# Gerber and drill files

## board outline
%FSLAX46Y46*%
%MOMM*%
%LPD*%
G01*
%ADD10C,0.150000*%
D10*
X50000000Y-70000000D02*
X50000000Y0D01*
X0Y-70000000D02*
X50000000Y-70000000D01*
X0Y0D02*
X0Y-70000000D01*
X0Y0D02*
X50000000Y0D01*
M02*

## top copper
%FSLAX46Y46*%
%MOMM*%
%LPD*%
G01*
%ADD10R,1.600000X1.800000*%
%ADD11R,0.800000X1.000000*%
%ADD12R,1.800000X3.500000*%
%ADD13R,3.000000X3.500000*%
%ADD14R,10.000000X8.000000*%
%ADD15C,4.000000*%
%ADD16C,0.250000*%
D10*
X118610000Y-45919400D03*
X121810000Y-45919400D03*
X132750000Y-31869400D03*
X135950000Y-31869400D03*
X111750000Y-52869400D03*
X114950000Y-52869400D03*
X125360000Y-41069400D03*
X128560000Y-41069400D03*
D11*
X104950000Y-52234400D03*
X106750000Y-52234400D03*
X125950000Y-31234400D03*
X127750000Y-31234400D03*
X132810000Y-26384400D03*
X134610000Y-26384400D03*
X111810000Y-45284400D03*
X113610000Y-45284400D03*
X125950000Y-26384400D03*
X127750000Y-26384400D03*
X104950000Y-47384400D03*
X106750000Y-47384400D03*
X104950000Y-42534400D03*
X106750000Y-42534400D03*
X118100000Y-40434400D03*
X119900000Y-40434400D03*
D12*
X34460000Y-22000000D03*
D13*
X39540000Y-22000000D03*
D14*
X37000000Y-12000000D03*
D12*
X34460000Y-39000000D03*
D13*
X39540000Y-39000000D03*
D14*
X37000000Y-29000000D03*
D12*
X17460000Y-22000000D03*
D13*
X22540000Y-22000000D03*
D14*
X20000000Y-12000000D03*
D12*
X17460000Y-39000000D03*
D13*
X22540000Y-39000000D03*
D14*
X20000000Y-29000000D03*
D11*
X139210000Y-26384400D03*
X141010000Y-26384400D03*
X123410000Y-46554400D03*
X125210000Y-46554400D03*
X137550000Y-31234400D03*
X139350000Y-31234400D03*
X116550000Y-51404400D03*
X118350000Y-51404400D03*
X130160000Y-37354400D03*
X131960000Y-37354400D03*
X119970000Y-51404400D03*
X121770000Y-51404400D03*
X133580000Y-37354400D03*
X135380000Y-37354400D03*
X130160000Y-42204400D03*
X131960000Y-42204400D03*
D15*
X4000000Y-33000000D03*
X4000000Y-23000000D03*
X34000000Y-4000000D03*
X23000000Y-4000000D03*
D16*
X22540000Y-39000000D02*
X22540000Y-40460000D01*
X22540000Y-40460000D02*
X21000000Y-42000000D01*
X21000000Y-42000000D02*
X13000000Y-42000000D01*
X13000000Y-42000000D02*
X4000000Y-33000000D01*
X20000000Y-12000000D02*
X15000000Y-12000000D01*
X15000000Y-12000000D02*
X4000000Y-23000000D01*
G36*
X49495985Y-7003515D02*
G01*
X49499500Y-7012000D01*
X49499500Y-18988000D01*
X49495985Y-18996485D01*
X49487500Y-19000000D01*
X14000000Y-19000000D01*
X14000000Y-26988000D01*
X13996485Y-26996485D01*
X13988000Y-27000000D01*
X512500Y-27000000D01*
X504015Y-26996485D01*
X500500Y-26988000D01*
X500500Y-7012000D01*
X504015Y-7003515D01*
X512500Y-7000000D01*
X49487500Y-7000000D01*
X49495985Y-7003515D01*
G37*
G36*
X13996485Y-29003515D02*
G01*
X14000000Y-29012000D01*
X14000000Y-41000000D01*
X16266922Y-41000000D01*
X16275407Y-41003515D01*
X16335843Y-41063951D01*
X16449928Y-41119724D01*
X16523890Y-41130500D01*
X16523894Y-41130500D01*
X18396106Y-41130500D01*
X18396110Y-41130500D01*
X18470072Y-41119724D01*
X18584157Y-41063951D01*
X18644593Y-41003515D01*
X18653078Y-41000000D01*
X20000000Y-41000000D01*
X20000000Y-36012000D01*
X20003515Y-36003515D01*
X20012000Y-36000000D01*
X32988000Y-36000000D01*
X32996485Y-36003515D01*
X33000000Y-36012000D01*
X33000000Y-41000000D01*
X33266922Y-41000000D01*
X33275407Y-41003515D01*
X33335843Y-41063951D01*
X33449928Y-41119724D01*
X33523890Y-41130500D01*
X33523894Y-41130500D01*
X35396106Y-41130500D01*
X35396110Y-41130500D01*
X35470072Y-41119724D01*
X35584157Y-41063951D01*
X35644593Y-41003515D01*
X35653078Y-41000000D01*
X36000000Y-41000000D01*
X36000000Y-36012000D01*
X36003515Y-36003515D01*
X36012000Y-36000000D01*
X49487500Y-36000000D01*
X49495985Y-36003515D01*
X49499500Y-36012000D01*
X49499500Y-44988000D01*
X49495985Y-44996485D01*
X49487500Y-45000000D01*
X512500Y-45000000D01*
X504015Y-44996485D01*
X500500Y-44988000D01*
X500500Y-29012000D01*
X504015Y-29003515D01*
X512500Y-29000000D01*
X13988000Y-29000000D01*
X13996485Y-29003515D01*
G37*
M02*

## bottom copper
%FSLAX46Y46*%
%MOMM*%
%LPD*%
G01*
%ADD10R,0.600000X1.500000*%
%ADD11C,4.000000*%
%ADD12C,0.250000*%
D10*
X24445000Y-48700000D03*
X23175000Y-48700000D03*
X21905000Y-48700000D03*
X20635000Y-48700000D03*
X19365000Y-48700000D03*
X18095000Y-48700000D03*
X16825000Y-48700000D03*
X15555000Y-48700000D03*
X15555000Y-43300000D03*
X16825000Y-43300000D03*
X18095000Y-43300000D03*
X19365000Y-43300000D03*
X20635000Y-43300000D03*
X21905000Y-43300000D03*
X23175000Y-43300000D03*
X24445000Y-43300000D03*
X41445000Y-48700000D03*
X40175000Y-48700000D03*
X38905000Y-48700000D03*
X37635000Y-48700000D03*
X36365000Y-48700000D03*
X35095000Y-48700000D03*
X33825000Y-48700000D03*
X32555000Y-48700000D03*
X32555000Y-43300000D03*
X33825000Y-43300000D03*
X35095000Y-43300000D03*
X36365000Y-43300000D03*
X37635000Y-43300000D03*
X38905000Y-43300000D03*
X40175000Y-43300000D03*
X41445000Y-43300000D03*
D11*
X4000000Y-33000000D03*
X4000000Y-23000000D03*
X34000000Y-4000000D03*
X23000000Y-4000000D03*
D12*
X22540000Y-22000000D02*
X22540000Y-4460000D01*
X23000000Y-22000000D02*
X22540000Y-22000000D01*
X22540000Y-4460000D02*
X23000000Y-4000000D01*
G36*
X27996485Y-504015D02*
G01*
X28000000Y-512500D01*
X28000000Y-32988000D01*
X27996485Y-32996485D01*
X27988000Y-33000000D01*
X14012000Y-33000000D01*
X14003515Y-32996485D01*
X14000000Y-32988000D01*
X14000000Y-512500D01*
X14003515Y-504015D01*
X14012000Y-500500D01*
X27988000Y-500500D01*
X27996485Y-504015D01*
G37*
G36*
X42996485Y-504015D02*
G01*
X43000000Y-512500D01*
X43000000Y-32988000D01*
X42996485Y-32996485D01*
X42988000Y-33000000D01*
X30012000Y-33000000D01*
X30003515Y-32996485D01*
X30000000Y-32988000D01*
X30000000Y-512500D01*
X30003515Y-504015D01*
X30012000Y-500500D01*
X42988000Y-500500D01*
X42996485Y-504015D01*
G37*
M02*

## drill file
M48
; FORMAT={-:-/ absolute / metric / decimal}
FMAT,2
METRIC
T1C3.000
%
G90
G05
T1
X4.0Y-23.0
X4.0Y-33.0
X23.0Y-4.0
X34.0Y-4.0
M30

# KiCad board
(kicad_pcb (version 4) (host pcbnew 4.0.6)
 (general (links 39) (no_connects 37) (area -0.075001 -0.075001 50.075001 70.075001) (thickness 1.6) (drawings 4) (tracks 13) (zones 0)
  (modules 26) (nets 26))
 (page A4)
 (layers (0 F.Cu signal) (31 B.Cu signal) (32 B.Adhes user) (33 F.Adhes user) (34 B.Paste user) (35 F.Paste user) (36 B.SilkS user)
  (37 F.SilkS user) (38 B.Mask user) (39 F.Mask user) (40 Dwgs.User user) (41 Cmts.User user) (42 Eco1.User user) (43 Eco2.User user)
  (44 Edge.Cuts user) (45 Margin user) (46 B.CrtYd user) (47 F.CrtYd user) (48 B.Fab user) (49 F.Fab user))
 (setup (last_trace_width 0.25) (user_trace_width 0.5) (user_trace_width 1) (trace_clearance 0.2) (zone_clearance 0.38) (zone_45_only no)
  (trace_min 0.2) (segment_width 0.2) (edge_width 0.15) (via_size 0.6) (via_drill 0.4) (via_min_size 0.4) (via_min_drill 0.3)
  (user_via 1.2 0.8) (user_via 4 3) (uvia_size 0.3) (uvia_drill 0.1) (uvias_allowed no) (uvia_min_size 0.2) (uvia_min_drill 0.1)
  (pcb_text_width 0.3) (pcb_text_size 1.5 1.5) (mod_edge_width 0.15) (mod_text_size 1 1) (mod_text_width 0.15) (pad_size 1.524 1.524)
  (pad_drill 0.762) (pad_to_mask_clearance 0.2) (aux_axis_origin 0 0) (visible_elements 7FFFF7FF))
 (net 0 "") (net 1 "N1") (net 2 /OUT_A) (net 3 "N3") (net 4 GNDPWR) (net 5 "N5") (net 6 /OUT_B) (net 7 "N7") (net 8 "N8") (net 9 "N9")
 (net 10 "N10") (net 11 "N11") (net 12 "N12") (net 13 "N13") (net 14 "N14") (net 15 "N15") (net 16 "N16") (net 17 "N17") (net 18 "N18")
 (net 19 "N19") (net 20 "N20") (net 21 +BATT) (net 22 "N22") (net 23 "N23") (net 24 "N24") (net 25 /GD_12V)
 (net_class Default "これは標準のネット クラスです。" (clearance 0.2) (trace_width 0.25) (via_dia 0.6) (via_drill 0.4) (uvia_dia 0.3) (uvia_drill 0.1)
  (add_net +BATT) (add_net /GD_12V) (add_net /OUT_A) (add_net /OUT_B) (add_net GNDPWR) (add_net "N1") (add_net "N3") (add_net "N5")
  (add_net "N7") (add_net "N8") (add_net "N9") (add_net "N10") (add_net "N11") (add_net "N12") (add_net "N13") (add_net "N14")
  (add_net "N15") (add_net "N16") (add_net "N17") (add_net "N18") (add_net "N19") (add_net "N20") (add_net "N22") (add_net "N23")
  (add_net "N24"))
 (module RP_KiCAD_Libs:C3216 (layer F.Cu) (at 120.21 45.9194)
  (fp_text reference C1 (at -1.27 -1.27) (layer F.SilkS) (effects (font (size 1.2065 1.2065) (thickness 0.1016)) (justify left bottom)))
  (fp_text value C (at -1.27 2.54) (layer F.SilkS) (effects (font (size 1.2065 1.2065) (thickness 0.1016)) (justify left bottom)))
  (pad 1 smd rect (at -1.6 0) (size 1.6 1.8) (layers F.Cu F.Paste F.Mask) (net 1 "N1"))
  (pad 2 smd rect (at 1.6 0) (size 1.6 1.8) (layers F.Cu F.Paste F.Mask) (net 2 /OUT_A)))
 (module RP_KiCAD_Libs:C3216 (layer F.Cu) (at 134.35 31.8694)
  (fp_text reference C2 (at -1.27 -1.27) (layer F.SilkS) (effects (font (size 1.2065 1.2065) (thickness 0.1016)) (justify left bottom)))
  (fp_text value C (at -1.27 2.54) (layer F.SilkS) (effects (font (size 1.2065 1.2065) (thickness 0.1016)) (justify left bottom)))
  (pad 1 smd rect (at -1.6 0) (size 1.6 1.8) (layers F.Cu F.Paste F.Mask) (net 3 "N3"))
  (pad 2 smd rect (at 1.6 0) (size 1.6 1.8) (layers F.Cu F.Paste F.Mask) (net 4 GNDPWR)))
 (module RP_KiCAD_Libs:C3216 (layer F.Cu) (at 113.35 52.8694)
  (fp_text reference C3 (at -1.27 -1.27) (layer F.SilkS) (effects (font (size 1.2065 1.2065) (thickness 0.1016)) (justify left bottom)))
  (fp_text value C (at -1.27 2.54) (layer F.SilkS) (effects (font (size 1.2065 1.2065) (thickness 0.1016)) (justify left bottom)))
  (pad 1 smd rect (at -1.6 0) (size 1.6 1.8) (layers F.Cu F.Paste F.Mask) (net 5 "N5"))
  (pad 2 smd rect (at 1.6 0) (size 1.6 1.8) (layers F.Cu F.Paste F.Mask) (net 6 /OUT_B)))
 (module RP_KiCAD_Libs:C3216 (layer F.Cu) (at 126.96 41.0694)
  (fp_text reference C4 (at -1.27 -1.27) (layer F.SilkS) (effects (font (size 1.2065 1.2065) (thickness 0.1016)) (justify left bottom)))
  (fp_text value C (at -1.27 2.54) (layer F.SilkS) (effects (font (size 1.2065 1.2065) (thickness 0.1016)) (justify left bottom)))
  (pad 1 smd rect (at -1.6 0) (size 1.6 1.8) (layers F.Cu F.Paste F.Mask) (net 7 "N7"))
  (pad 2 smd rect (at 1.6 0) (size 1.6 1.8) (layers F.Cu F.Paste F.Mask) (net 4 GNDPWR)))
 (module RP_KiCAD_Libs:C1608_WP (layer F.Cu) (at 105.85 52.2344)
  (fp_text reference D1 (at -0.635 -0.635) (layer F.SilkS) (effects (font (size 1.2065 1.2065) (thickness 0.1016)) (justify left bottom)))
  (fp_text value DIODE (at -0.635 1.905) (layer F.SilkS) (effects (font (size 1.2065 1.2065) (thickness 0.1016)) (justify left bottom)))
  (pad 1 smd rect (at -0.9 0) (size 0.8 1) (layers F.Cu F.Paste F.Mask) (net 1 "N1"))
  (pad 2 smd rect (at 0.9 0) (size 0.8 1) (layers F.Cu F.Paste F.Mask) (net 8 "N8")))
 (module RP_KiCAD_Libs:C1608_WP (layer F.Cu) (at 126.85 31.2344)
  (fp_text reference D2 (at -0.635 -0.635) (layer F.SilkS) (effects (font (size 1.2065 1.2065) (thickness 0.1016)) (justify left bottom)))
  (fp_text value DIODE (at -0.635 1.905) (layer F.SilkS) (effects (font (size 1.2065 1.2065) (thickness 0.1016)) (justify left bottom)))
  (pad 1 smd rect (at -0.9 0) (size 0.8 1) (layers F.Cu F.Paste F.Mask) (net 3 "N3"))
  (pad 2 smd rect (at 0.9 0) (size 0.8 1) (layers F.Cu F.Paste F.Mask) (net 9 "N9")))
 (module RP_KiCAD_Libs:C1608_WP (layer F.Cu) (at 133.71 26.3844)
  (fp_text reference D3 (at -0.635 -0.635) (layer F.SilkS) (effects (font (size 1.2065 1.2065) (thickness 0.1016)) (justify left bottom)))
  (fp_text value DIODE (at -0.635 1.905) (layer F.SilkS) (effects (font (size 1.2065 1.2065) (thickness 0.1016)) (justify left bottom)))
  (pad 1 smd rect (at -0.9 0) (size 0.8 1) (layers F.Cu F.Paste F.Mask) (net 5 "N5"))
  (pad 2 smd rect (at 0.9 0) (size 0.8 1) (layers F.Cu F.Paste F.Mask) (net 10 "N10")))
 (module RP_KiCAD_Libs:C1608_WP (layer F.Cu) (at 112.71 45.2844)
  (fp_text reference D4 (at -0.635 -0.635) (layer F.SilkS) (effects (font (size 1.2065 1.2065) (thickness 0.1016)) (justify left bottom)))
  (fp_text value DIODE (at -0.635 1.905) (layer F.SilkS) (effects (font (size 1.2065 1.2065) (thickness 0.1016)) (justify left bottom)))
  (pad 1 smd rect (at -0.9 0) (size 0.8 1) (layers F.Cu F.Paste F.Mask) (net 7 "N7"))
  (pad 2 smd rect (at 0.9 0) (size 0.8 1) (layers F.Cu F.Paste F.Mask) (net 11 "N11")))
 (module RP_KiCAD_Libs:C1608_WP (layer F.Cu) (at 126.85 26.3844)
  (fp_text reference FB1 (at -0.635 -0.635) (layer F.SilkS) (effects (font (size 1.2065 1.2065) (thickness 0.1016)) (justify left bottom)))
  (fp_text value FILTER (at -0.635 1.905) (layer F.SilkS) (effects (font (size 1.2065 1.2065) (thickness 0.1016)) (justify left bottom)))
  (pad 1 smd rect (at -0.9 0) (size 0.8 1) (layers F.Cu F.Paste F.Mask) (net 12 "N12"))
  (pad 2 smd rect (at 0.9 0) (size 0.8 1) (layers F.Cu F.Paste F.Mask) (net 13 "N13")))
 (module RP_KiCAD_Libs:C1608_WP (layer F.Cu) (at 105.85 47.3844)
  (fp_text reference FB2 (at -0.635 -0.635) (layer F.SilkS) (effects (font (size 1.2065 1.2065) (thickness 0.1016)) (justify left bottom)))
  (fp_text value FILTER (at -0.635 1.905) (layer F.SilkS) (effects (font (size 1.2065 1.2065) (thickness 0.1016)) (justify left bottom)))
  (pad 1 smd rect (at -0.9 0) (size 0.8 1) (layers F.Cu F.Paste F.Mask) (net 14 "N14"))
  (pad 2 smd rect (at 0.9 0) (size 0.8 1) (layers F.Cu F.Paste F.Mask) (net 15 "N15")))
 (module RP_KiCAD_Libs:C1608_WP (layer F.Cu) (at 105.85 42.5344)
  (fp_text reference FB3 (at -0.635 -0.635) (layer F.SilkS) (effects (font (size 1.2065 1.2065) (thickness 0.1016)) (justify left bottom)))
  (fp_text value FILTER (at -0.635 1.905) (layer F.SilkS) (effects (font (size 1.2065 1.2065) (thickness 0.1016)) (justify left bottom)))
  (pad 1 smd rect (at -0.9 0) (size 0.8 1) (layers F.Cu F.Paste F.Mask) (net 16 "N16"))
  (pad 2 smd rect (at 0.9 0) (size 0.8 1) (layers F.Cu F.Paste F.Mask) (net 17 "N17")))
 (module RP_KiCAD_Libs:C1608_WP (layer F.Cu) (at 119 40.4344)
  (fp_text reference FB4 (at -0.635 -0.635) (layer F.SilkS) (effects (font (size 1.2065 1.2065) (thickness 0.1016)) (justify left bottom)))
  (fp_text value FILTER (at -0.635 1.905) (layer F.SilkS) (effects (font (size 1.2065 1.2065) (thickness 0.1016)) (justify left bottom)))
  (pad 1 smd rect (at -0.9 0) (size 0.8 1) (layers F.Cu F.Paste F.Mask) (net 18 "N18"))
  (pad 2 smd rect (at 0.9 0) (size 0.8 1) (layers F.Cu F.Paste F.Mask) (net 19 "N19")))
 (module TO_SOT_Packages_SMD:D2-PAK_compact (layer F.Cu) (at 37 19)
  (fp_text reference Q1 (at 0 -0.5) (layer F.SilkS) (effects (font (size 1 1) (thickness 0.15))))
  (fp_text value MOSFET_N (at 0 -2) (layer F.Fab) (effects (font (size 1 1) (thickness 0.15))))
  (pad G smd rect (at -2.54 3) (size 1.8 3.5) (layers F.Cu F.Paste F.Mask) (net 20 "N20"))
  (pad S smd rect (at 2.54 3) (size 3 3.5) (layers F.Cu F.Paste F.Mask) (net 2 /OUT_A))
  (pad D smd rect (at 0 -7) (size 10 8) (layers F.Cu F.Paste F.Mask) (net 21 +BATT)))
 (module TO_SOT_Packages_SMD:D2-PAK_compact (layer F.Cu) (at 37 36)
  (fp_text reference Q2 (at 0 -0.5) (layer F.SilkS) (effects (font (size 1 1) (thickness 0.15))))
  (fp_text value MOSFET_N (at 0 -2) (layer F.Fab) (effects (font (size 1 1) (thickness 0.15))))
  (pad G smd rect (at -2.54 3) (size 1.8 3.5) (layers F.Cu F.Paste F.Mask) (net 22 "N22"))
  (pad S smd rect (at 2.54 3) (size 3 3.5) (layers F.Cu F.Paste F.Mask) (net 4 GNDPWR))
  (pad D smd rect (at 0 -7) (size 10 8) (layers F.Cu F.Paste F.Mask) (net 2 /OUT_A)))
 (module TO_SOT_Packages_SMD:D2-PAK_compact (layer F.Cu) (at 20 19)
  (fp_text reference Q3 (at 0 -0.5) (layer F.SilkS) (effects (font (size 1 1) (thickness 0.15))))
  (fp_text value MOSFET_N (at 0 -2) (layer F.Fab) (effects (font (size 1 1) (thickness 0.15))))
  (pad G smd rect (at -2.54 3) (size 1.8 3.5) (layers F.Cu F.Paste F.Mask) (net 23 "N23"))
  (pad S smd rect (at 2.54 3) (size 3 3.5) (layers F.Cu F.Paste F.Mask) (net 6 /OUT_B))
  (pad D smd rect (at 0 -7) (size 10 8) (layers F.Cu F.Paste F.Mask) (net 21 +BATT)))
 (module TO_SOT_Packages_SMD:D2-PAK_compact (layer F.Cu) (at 20 36)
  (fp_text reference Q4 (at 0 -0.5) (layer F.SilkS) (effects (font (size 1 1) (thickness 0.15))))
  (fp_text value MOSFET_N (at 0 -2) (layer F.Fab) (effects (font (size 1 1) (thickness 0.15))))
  (pad G smd rect (at -2.54 3) (size 1.8 3.5) (layers F.Cu F.Paste F.Mask) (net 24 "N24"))
  (pad S smd rect (at 2.54 3) (size 3 3.5) (layers F.Cu F.Paste F.Mask) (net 4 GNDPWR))
  (pad D smd rect (at 0 -7) (size 10 8) (layers F.Cu F.Paste F.Mask) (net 6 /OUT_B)))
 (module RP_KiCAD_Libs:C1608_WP (layer F.Cu) (at 140.11 26.3844)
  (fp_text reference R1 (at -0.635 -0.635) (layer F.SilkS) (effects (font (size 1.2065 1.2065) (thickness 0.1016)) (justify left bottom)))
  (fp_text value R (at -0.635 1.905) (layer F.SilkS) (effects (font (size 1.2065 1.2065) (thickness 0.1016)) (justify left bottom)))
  (pad 1 smd rect (at -0.9 0) (size 0.8 1) (layers F.Cu F.Paste F.Mask) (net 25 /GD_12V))
  (pad 2 smd rect (at 0.9 0) (size 0.8 1) (layers F.Cu F.Paste F.Mask) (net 8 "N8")))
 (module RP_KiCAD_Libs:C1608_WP (layer F.Cu) (at 124.31 46.5544)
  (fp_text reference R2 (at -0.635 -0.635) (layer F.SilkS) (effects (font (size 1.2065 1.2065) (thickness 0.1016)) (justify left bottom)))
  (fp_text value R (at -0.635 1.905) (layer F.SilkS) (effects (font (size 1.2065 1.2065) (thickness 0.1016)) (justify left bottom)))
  (pad 1 smd rect (at -0.9 0) (size 0.8 1) (layers F.Cu F.Paste F.Mask) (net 25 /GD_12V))
  (pad 2 smd rect (at 0.9 0) (size 0.8 1) (layers F.Cu F.Paste F.Mask) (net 9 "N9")))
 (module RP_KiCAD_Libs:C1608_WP (layer F.Cu) (at 138.45 31.2344)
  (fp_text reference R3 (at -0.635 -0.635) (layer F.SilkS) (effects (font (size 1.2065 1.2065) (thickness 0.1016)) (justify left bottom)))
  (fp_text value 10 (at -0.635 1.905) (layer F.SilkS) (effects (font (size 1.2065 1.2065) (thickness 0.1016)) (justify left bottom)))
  (pad 1 smd rect (at -0.9 0) (size 0.8 1) (layers F.Cu F.Paste F.Mask) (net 20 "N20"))
  (pad 2 smd rect (at 0.9 0) (size 0.8 1) (layers F.Cu F.Paste F.Mask) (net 13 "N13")))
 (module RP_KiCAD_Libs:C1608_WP (layer F.Cu) (at 117.45 51.4044)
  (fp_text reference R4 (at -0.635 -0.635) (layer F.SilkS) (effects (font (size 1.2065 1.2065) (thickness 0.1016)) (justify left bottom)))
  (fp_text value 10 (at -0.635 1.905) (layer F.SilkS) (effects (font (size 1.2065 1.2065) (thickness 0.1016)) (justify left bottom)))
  (pad 1 smd rect (at -0.9 0) (size 0.8 1) (layers F.Cu F.Paste F.Mask) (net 22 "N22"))
  (pad 2 smd rect (at 0.9 0) (size 0.8 1) (layers F.Cu F.Paste F.Mask) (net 15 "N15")))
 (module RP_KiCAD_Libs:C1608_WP (layer F.Cu) (at 131.06 37.3544)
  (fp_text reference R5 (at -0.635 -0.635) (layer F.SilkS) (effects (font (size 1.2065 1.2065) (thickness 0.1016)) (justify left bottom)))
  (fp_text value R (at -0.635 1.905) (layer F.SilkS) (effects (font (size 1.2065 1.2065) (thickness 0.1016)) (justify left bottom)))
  (pad 1 smd rect (at -0.9 0) (size 0.8 1) (layers F.Cu F.Paste F.Mask) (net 25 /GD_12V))
  (pad 2 smd rect (at 0.9 0) (size 0.8 1) (layers F.Cu F.Paste F.Mask) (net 10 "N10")))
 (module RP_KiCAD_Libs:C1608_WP (layer F.Cu) (at 120.87 51.4044)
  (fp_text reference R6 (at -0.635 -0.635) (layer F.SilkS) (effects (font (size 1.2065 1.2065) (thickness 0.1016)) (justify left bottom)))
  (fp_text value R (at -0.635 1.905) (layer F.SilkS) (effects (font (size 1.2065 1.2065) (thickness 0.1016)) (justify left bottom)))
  (pad 1 smd rect (at -0.9 0) (size 0.8 1) (layers F.Cu F.Paste F.Mask) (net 25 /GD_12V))
  (pad 2 smd rect (at 0.9 0) (size 0.8 1) (layers F.Cu F.Paste F.Mask) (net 11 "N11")))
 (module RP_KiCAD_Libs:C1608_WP (layer F.Cu) (at 134.48 37.3544)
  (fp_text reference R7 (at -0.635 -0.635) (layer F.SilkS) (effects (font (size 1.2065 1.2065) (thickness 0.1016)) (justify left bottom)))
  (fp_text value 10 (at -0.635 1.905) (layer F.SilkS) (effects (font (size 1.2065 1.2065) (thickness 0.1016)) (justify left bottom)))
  (pad 1 smd rect (at -0.9 0) (size 0.8 1) (layers F.Cu F.Paste F.Mask) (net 23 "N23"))
  (pad 2 smd rect (at 0.9 0) (size 0.8 1) (layers F.Cu F.Paste F.Mask) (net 17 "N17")))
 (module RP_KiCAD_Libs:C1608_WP (layer F.Cu) (at 131.06 42.2044)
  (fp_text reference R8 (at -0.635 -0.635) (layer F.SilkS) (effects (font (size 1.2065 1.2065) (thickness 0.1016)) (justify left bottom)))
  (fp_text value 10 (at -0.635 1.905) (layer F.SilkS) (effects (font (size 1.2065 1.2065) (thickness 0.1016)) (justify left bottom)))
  (pad 1 smd rect (at -0.9 0) (size 0.8 1) (layers F.Cu F.Paste F.Mask) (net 24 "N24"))
  (pad 2 smd rect (at 0.9 0) (size 0.8 1) (layers F.Cu F.Paste F.Mask) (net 19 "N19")))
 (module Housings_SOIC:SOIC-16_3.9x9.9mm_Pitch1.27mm (layer B.Cu) (at 20 46 90)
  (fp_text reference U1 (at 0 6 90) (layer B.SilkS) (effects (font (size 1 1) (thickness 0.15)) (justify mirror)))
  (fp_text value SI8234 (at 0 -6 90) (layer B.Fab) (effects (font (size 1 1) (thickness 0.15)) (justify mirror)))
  (pad 1 smd rect (at -2.7 4.445 90) (size 1.5 0.6) (layers B.Cu B.Paste B.Mask))
  (pad 2 smd rect (at -2.7 3.175 90) (size 1.5 0.6) (layers B.Cu B.Paste B.Mask))
  (pad 3 smd rect (at -2.7 1.905 90) (size 1.5 0.6) (layers B.Cu B.Paste B.Mask))
  (pad 4 smd rect (at -2.7 0.635 90) (size 1.5 0.6) (layers B.Cu B.Paste B.Mask))
  (pad 5 smd rect (at -2.7 -0.635 90) (size 1.5 0.6) (layers B.Cu B.Paste B.Mask))
  (pad 6 smd rect (at -2.7 -1.905 90) (size 1.5 0.6) (layers B.Cu B.Paste B.Mask))
  (pad 7 smd rect (at -2.7 -3.175 90) (size 1.5 0.6) (layers B.Cu B.Paste B.Mask))
  (pad 8 smd rect (at -2.7 -4.445 90) (size 1.5 0.6) (layers B.Cu B.Paste B.Mask))
  (pad 9 smd rect (at 2.7 -4.445 90) (size 1.5 0.6) (layers B.Cu B.Paste B.Mask) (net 4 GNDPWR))
  (pad 10 smd rect (at 2.7 -3.175 90) (size 1.5 0.6) (layers B.Cu B.Paste B.Mask) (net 14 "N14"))
  (pad 11 smd rect (at 2.7 -1.905 90) (size 1.5 0.6) (layers B.Cu B.Paste B.Mask) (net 3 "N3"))
  (pad 12 smd rect (at 2.7 -0.635 90) (size 1.5 0.6) (layers B.Cu B.Paste B.Mask))
  (pad 13 smd rect (at 2.7 0.635 90) (size 1.5 0.6) (layers B.Cu B.Paste B.Mask))
  (pad 14 smd rect (at 2.7 1.905 90) (size 1.5 0.6) (layers B.Cu B.Paste B.Mask) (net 2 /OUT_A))
  (pad 15 smd rect (at 2.7 3.175 90) (size 1.5 0.6) (layers B.Cu B.Paste B.Mask) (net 12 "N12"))
  (pad 16 smd rect (at 2.7 4.445 90) (size 1.5 0.6) (layers B.Cu B.Paste B.Mask) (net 1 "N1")))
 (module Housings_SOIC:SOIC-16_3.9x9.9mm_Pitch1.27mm (layer B.Cu) (at 37 46 90)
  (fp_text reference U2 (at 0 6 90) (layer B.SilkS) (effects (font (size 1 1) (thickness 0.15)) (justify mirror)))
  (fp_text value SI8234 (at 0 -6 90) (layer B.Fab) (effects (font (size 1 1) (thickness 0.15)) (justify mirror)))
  (pad 1 smd rect (at -2.7 4.445 90) (size 1.5 0.6) (layers B.Cu B.Paste B.Mask))
  (pad 2 smd rect (at -2.7 3.175 90) (size 1.5 0.6) (layers B.Cu B.Paste B.Mask))
  (pad 3 smd rect (at -2.7 1.905 90) (size 1.5 0.6) (layers B.Cu B.Paste B.Mask))
  (pad 4 smd rect (at -2.7 0.635 90) (size 1.5 0.6) (layers B.Cu B.Paste B.Mask))
  (pad 5 smd rect (at -2.7 -0.635 90) (size 1.5 0.6) (layers B.Cu B.Paste B.Mask))
  (pad 6 smd rect (at -2.7 -1.905 90) (size 1.5 0.6) (layers B.Cu B.Paste B.Mask))
  (pad 7 smd rect (at -2.7 -3.175 90) (size 1.5 0.6) (layers B.Cu B.Paste B.Mask))
  (pad 8 smd rect (at -2.7 -4.445 90) (size 1.5 0.6) (layers B.Cu B.Paste B.Mask))
  (pad 9 smd rect (at 2.7 -4.445 90) (size 1.5 0.6) (layers B.Cu B.Paste B.Mask) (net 4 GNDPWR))
  (pad 10 smd rect (at 2.7 -3.175 90) (size 1.5 0.6) (layers B.Cu B.Paste B.Mask) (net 18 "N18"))
  (pad 11 smd rect (at 2.7 -1.905 90) (size 1.5 0.6) (layers B.Cu B.Paste B.Mask) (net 7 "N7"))
  (pad 12 smd rect (at 2.7 -0.635 90) (size 1.5 0.6) (layers B.Cu B.Paste B.Mask))
  (pad 13 smd rect (at 2.7 0.635 90) (size 1.5 0.6) (layers B.Cu B.Paste B.Mask))
  (pad 14 smd rect (at 2.7 1.905 90) (size 1.5 0.6) (layers B.Cu B.Paste B.Mask) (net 6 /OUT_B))
  (pad 15 smd rect (at 2.7 3.175 90) (size 1.5 0.6) (layers B.Cu B.Paste B.Mask) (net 16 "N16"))
  (pad 16 smd rect (at 2.7 4.445 90) (size 1.5 0.6) (layers B.Cu B.Paste B.Mask) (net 5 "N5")))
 (gr_line (start 50 70) (end 50 0) (angle 90) (layer Edge.Cuts) (width 0.15))
 (gr_line (start 0 70) (end 50 70) (angle 90) (layer Edge.Cuts) (width 0.15))
 (gr_line (start 0 0) (end 0 70) (angle 90) (layer Edge.Cuts) (width 0.15))
 (gr_line (start 0 0) (end 50 0) (angle 90) (layer Edge.Cuts) (width 0.15))
 (segment (start 22.54 39) (end 22.54 40.46) (width 0.25) (layer F.Cu) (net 4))
 (segment (start 22.54 40.46) (end 21 42) (width 0.25) (layer F.Cu) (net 4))
 (segment (start 21 42) (end 13 42) (width 0.25) (layer F.Cu) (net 4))
 (segment (start 13 42) (end 4 33) (width 0.25) (layer F.Cu) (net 4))
 (via (at 4 33) (size 4) (drill 3) (layers F.Cu B.Cu) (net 4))
 (segment (start 20 12) (end 15 12) (width 0.25) (layer F.Cu) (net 21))
 (segment (start 15 12) (end 4 23) (width 0.25) (layer F.Cu) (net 21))
 (via (at 4 23) (size 4) (drill 3) (layers F.Cu B.Cu) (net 21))
 (via (at 34 4) (size 4) (drill 3) (layers F.Cu B.Cu) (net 2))
 (segment (start 22.54 22) (end 22.54 4.46) (width 0.25) (layer B.Cu) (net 6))
 (segment (start 23 22) (end 22.54 22) (width 0.25) (layer B.Cu) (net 6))
 (via (at 23 4) (size 4) (drill 3) (layers F.Cu B.Cu) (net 6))
 (segment (start 22.54 4.46) (end 23 4) (width 0.25) (layer B.Cu) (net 6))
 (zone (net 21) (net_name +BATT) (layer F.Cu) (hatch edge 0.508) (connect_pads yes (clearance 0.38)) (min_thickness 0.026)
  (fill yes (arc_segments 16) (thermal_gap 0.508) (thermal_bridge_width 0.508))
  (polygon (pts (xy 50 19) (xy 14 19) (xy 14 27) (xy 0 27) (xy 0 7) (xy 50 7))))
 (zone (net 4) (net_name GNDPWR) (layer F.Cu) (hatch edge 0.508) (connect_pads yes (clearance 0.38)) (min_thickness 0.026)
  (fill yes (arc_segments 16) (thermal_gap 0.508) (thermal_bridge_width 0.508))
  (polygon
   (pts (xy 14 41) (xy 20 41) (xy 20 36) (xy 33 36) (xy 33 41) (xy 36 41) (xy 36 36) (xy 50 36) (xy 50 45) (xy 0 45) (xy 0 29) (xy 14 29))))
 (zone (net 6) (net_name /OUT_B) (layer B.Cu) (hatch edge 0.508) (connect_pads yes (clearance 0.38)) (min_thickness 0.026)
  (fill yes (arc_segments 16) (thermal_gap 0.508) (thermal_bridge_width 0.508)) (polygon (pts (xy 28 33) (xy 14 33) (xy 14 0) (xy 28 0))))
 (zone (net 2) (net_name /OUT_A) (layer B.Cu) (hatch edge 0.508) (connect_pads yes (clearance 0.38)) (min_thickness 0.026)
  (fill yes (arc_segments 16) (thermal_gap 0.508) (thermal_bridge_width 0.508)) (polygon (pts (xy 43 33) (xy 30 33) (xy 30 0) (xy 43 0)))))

